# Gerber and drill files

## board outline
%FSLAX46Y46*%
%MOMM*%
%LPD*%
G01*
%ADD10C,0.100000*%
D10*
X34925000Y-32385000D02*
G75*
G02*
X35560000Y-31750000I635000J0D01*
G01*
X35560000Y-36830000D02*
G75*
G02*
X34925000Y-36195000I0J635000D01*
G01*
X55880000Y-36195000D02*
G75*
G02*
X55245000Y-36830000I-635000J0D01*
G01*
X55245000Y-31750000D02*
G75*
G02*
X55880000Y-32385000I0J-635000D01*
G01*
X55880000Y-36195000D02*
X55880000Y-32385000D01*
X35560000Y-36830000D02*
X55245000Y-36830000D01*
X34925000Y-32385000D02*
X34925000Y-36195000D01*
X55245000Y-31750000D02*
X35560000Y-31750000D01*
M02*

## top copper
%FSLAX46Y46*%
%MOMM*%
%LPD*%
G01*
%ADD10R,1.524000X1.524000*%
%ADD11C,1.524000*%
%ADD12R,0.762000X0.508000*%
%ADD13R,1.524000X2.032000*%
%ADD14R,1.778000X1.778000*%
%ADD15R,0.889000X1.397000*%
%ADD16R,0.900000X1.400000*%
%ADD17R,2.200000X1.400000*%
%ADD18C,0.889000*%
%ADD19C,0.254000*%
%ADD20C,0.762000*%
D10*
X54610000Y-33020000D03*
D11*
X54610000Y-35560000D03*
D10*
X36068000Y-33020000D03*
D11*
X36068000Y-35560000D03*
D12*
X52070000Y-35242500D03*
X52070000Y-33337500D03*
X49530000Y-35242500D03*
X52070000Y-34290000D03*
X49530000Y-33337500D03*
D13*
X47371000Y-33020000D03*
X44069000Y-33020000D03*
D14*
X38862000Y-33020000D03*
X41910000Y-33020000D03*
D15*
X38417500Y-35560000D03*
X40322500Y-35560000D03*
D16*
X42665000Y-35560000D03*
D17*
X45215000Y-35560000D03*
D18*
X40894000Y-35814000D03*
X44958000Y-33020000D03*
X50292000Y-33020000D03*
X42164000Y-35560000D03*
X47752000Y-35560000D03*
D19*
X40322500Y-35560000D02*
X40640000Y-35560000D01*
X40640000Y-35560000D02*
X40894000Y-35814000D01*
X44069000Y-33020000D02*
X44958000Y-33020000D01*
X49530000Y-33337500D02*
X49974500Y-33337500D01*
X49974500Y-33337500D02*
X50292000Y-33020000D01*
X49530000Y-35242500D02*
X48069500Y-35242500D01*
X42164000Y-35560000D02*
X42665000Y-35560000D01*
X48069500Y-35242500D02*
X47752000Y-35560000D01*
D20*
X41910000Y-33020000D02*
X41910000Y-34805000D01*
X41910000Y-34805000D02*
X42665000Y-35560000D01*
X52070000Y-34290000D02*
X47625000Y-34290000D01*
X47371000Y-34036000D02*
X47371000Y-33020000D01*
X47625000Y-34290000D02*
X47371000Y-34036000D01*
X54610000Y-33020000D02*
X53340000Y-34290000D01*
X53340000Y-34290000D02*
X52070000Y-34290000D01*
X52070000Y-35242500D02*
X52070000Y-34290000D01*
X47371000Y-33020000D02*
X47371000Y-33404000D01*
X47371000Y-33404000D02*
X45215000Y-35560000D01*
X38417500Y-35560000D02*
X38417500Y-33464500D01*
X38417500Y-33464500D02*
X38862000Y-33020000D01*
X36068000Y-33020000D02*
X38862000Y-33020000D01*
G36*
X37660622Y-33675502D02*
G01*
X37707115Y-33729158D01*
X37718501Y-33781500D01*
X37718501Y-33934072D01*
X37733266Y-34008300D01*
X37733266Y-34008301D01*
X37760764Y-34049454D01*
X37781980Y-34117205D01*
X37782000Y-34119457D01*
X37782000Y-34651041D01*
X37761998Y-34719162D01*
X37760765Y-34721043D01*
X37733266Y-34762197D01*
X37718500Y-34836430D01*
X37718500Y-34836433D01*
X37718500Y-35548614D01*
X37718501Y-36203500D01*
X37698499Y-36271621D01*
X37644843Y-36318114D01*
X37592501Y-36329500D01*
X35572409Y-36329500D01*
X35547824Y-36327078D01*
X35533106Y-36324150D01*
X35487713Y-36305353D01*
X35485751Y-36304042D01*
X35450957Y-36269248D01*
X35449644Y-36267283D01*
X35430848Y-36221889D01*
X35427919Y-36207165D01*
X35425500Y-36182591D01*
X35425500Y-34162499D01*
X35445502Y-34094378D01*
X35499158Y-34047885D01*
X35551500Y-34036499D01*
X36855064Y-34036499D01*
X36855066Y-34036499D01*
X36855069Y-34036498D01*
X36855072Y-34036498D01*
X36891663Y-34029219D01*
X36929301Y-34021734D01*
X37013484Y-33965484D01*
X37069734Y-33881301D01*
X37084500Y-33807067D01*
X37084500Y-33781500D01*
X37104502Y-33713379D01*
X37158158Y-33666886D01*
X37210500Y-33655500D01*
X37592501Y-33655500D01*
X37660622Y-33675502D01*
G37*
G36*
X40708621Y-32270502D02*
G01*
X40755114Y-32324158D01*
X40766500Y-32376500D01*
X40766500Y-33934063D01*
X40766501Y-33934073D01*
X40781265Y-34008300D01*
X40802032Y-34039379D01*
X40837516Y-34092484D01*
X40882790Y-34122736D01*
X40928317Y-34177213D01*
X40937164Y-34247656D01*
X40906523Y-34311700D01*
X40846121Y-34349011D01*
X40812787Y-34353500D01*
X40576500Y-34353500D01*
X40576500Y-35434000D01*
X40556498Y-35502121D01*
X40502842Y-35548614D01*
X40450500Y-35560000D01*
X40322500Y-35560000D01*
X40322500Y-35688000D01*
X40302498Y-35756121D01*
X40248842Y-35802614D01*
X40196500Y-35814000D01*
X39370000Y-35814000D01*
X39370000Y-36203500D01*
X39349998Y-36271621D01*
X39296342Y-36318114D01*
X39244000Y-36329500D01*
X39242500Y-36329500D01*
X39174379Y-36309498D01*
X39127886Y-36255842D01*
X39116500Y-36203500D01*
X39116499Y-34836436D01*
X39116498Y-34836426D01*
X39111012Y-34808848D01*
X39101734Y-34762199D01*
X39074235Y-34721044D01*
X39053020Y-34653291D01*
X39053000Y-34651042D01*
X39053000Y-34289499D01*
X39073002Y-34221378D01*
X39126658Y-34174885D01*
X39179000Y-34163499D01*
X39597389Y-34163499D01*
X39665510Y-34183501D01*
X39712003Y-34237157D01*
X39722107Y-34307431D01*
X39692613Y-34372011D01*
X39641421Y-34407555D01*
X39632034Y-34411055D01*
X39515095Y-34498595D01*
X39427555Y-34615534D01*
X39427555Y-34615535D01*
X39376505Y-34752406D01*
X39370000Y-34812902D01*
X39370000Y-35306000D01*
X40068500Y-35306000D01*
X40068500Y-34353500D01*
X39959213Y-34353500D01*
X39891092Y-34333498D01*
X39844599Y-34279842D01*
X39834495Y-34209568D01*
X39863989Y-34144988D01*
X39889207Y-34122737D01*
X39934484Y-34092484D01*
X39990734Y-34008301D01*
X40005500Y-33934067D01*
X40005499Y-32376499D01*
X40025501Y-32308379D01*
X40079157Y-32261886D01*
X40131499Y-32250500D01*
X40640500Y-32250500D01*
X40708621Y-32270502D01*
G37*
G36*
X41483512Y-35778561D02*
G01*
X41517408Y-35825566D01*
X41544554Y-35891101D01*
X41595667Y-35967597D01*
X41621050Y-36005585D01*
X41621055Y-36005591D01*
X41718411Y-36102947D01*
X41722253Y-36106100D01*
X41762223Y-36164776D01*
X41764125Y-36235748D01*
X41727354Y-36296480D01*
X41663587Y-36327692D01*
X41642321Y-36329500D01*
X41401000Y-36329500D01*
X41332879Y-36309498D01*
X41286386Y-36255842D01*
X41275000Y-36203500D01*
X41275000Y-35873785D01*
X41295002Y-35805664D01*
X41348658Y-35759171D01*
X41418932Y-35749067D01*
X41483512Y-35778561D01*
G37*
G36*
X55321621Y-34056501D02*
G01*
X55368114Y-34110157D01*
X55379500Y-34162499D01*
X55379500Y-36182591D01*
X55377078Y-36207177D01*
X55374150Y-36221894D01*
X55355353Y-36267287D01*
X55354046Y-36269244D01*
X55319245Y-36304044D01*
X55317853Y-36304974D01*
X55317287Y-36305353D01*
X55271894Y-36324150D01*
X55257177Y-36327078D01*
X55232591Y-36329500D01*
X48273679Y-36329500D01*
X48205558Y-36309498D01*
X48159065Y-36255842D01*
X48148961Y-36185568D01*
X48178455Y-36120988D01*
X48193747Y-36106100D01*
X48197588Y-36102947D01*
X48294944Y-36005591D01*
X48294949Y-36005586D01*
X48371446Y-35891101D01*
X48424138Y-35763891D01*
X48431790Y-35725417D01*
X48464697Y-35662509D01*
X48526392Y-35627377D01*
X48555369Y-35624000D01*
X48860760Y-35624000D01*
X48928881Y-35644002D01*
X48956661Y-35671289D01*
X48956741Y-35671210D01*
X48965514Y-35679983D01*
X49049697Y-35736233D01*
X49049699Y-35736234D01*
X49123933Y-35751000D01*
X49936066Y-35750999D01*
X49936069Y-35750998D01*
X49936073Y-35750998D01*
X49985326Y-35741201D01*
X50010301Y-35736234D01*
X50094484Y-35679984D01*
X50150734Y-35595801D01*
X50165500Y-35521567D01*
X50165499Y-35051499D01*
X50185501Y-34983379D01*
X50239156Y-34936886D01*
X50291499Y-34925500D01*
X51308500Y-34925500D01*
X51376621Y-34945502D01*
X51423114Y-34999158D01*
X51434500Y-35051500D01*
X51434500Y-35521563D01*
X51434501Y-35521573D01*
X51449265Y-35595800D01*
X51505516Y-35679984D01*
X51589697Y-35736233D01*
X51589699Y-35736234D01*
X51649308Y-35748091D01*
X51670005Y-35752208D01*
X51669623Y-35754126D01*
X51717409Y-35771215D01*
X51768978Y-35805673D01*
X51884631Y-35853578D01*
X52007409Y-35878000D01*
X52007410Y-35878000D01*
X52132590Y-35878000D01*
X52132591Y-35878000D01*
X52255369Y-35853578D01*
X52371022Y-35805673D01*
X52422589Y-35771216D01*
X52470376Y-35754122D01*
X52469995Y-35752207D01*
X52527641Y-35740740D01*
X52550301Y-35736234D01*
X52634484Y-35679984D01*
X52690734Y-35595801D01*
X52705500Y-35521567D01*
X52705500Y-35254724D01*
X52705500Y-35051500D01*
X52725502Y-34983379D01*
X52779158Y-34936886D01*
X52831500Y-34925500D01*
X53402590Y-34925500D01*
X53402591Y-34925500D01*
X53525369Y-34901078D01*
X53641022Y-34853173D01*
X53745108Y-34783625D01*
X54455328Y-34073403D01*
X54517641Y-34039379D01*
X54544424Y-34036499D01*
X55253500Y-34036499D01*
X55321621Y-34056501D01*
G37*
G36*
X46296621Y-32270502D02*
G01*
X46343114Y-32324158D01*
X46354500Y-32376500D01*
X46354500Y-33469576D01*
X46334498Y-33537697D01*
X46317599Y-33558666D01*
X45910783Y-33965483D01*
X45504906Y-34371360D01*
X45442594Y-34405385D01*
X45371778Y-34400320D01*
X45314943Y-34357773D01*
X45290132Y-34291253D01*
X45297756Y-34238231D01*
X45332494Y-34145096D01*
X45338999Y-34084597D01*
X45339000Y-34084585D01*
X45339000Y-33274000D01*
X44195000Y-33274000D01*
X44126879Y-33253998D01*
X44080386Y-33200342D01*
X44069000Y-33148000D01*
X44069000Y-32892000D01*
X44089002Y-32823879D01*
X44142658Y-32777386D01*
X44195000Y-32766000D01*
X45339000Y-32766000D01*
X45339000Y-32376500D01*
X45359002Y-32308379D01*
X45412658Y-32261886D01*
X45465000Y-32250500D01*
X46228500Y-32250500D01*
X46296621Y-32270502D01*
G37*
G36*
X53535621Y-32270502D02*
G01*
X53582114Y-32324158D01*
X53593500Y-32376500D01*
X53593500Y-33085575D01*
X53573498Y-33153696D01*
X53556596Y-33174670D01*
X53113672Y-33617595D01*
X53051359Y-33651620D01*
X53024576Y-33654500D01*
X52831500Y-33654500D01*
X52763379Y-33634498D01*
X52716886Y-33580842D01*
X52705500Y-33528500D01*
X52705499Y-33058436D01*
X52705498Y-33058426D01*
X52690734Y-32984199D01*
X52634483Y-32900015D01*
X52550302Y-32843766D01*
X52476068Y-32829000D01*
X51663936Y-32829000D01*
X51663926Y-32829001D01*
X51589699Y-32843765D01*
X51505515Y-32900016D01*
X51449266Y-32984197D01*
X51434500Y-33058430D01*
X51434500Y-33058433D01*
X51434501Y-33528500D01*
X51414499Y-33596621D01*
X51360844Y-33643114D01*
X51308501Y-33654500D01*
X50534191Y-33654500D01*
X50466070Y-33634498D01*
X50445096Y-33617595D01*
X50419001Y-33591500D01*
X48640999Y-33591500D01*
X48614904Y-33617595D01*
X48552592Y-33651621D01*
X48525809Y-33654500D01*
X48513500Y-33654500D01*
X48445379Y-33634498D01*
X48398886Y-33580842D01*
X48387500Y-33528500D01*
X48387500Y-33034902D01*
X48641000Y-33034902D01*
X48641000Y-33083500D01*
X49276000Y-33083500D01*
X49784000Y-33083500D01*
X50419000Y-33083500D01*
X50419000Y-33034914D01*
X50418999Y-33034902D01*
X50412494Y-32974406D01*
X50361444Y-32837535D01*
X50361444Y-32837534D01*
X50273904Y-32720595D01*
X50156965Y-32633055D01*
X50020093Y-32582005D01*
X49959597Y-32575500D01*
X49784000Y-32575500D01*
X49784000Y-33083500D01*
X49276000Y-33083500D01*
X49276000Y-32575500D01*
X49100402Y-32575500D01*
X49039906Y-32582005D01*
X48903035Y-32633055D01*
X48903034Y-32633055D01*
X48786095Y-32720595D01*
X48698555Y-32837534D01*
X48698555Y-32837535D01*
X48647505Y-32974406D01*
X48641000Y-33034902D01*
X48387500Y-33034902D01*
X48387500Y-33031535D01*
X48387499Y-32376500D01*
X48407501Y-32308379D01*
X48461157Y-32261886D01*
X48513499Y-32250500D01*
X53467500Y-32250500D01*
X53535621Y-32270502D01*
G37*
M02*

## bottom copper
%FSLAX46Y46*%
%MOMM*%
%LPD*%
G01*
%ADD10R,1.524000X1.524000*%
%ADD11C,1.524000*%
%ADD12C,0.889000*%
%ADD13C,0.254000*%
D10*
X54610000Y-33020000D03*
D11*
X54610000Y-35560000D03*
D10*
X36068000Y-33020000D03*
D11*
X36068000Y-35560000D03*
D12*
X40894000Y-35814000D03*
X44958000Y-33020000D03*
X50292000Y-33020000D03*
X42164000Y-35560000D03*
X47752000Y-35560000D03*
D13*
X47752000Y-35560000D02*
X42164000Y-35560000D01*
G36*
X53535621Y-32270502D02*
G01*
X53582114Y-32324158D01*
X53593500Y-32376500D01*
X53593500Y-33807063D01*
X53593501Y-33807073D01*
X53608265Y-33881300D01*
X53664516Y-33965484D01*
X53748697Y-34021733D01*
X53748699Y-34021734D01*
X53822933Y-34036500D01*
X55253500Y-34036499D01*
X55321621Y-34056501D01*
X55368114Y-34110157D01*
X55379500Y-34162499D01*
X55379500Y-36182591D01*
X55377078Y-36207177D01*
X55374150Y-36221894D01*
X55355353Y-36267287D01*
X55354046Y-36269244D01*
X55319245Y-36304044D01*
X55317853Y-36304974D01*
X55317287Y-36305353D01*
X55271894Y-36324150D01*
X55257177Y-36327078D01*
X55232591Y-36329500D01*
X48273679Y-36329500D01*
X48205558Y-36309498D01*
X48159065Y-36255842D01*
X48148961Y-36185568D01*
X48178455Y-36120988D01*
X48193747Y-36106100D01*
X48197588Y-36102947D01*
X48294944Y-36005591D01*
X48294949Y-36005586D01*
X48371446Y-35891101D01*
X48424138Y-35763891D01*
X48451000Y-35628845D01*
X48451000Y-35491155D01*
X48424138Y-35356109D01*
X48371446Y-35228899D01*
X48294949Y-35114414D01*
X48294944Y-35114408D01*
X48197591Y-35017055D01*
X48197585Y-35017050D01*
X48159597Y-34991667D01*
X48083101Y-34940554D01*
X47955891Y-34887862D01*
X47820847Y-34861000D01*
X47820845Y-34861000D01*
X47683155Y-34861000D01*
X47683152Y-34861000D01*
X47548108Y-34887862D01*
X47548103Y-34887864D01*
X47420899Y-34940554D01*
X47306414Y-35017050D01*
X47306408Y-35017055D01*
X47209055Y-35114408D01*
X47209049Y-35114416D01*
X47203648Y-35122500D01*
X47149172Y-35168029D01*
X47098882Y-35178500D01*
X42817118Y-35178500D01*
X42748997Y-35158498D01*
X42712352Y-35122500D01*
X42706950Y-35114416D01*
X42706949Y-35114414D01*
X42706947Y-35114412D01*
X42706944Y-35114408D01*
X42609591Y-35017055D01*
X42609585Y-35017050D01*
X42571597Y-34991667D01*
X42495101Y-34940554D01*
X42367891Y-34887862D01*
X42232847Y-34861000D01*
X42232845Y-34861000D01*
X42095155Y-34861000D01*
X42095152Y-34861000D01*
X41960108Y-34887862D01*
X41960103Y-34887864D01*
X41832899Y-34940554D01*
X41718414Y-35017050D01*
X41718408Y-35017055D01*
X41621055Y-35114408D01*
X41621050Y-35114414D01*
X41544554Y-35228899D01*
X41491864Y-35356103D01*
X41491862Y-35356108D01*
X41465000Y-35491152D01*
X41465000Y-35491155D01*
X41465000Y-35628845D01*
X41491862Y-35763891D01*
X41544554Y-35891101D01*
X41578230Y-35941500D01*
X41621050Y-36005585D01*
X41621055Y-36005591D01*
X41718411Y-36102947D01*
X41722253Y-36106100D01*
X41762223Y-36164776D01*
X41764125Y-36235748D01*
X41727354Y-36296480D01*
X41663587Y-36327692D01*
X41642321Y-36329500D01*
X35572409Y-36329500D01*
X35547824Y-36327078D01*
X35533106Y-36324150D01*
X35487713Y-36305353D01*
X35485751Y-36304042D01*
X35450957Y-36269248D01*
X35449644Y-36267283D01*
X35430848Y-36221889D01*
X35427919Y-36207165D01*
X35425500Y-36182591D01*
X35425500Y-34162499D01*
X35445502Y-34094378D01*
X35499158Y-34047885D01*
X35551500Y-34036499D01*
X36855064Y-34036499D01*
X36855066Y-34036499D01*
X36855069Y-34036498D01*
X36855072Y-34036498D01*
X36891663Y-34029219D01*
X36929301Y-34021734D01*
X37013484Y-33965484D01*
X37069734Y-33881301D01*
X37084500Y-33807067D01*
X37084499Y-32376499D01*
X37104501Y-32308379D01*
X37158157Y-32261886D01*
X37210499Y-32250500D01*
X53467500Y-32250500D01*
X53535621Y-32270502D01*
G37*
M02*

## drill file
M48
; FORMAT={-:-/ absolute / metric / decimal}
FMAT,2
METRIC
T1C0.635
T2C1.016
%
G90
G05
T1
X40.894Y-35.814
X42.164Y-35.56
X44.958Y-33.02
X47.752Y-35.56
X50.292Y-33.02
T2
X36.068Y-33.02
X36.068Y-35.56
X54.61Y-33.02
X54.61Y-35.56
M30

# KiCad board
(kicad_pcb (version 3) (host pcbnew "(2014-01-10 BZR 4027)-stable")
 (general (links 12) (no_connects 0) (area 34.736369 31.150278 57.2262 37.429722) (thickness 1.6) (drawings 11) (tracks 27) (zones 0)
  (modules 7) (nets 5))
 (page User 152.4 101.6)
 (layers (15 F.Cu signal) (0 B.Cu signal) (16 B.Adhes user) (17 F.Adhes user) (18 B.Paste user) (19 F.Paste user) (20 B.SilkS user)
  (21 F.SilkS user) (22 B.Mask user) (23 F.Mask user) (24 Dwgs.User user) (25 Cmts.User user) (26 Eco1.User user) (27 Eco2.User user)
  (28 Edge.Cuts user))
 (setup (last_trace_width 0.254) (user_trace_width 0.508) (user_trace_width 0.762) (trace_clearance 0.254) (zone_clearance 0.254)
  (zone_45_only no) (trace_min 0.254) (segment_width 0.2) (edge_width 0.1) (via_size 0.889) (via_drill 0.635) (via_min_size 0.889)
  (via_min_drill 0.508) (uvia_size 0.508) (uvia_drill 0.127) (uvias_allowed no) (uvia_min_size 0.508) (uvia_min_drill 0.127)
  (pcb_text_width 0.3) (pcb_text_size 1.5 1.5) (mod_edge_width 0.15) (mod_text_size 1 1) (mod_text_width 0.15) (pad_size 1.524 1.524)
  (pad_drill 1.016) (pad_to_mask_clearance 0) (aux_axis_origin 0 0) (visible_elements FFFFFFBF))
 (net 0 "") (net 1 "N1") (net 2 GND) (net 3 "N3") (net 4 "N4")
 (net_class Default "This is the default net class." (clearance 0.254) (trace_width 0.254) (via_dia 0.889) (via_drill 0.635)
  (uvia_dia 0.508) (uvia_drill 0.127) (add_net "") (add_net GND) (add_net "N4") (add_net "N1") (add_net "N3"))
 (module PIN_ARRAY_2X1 (layer F.Cu) (at 54.61 34.29 270)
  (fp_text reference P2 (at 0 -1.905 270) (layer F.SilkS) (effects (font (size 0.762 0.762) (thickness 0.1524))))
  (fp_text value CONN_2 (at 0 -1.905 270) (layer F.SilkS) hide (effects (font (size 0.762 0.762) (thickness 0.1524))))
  (pad 1 thru_hole rect (at -1.27 0 270) (size 1.524 1.524) (drill 1.016) (layers *.Cu *.Mask F.SilkS) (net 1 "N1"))
  (pad 2 thru_hole circle (at 1.27 0 270) (size 1.524 1.524) (drill 1.016) (layers *.Cu *.Mask F.SilkS) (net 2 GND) (zone_connect 2)))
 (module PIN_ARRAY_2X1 (layer F.Cu) (at 36.068 34.29 270)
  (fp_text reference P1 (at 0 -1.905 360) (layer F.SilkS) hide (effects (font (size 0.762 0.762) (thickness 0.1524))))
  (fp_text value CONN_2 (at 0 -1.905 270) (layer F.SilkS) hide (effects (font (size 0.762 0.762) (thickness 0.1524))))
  (pad 1 thru_hole rect (at -1.27 0 270) (size 1.524 1.524) (drill 1.016) (layers *.Cu *.Mask F.SilkS) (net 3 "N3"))
  (pad 2 thru_hole circle (at 1.27 0 270) (size 1.524 1.524) (drill 1.016) (layers *.Cu *.Mask F.SilkS) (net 2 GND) (zone_connect 2)))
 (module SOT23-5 (layer F.Cu) (at 50.8 34.29 90)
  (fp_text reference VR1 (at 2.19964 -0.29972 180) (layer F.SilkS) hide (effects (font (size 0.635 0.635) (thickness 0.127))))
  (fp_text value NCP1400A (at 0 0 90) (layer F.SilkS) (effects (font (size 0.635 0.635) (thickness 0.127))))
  (pad 1 smd rect (at -0.9525 1.27 90) (size 0.508 0.762) (layers F.Cu F.Paste F.Mask) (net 1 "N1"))
  (pad 3 smd rect (at 0.9525 1.27 90) (size 0.508 0.762) (layers F.Cu F.Paste F.Mask))
  (pad 5 smd rect (at -0.9525 -1.27 90) (size 0.508 0.762) (layers F.Cu F.Paste F.Mask) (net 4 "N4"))
  (pad 2 smd rect (at 0 1.27 90) (size 0.508 0.762) (layers F.Cu F.Paste F.Mask) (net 1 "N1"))
  (pad 4 smd rect (at 0.9525 -1.27 90) (size 0.508 0.762) (layers F.Cu F.Paste F.Mask) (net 2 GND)))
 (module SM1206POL (layer F.Cu) (at 45.72 33.02 180)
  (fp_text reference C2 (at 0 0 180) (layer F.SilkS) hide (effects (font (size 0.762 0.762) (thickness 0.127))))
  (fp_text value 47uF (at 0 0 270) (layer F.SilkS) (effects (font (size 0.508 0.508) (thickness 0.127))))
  (pad 1 smd rect (at -1.651 0 180) (size 1.524 2.032) (layers F.Cu F.Paste F.Mask) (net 1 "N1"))
  (pad 2 smd rect (at 1.651 0 180) (size 1.524 2.032) (layers F.Cu F.Paste F.Mask) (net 2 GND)))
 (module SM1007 (layer F.Cu) (at 40.386 33.02)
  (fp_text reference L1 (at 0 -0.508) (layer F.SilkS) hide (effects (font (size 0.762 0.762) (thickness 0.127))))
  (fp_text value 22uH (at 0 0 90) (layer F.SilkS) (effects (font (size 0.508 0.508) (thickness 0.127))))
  (pad 1 smd rect (at -1.524 0) (size 1.778 1.778) (layers F.Cu F.Paste F.Mask) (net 3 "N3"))
  (pad 2 smd rect (at 1.524 0) (size 1.778 1.778) (layers F.Cu F.Paste F.Mask) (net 4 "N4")))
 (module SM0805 (layer F.Cu) (at 39.37 35.56)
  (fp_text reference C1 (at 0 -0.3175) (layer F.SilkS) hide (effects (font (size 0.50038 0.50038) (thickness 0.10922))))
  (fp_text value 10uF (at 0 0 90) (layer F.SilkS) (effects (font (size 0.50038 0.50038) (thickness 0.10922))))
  (pad 1 smd rect (at -0.9525 0) (size 0.889 1.397) (layers F.Cu F.Paste F.Mask) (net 3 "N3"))
  (pad 2 smd rect (at 0.9525 0) (size 0.889 1.397) (layers F.Cu F.Paste F.Mask) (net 2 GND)))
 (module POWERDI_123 (layer F.Cu) (at 43.815 35.56)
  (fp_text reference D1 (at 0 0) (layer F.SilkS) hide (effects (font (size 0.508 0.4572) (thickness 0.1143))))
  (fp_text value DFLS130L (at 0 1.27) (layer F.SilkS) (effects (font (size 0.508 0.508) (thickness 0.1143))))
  (pad 1 smd rect (at -1.15 0) (size 0.9 1.4) (layers F.Cu F.Paste F.Mask) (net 4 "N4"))
  (pad 2 smd rect (at 1.4 0) (size 2.2 1.4) (layers F.Cu F.Paste F.Mask) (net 1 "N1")))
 (gr_arc (start 35.56 32.385) (end 34.925 32.385) (angle 90) (layer Edge.Cuts) (width 0.1))
 (gr_arc (start 35.56 36.195) (end 35.56 36.83) (angle 90) (layer Edge.Cuts) (width 0.1))
 (gr_arc (start 55.245 36.195) (end 55.88 36.195) (angle 90) (layer Edge.Cuts) (width 0.1))
 (gr_arc (start 55.245 32.385) (end 55.245 31.75) (angle 90) (layer Edge.Cuts) (width 0.1))
 (gr_line (start 55.88 36.195) (end 55.88 32.385) (angle 90) (layer Edge.Cuts) (width 0.1))
 (gr_line (start 35.56 36.83) (end 55.245 36.83) (angle 90) (layer Edge.Cuts) (width 0.1))
 (gr_line (start 34.925 32.385) (end 34.925 36.195) (angle 90) (layer Edge.Cuts) (width 0.1))
 (gr_line (start 55.245 31.75) (end 35.56 31.75) (angle 90) (layer Edge.Cuts) (width 0.1))
 (segment (start 40.3225 35.56) (end 40.64 35.56) (width 0.254) (layer F.Cu) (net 2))
 (via (at 40.894 35.814) (size 0.889) (layers F.Cu B.Cu) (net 2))
 (segment (start 40.64 35.56) (end 40.894 35.814) (width 0.254) (layer F.Cu) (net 2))
 (segment (start 44.069 33.02) (end 44.958 33.02) (width 0.254) (layer F.Cu) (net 2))
 (via (at 44.958 33.02) (size 0.889) (layers F.Cu B.Cu) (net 2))
 (segment (start 49.53 33.3375) (end 49.9745 33.3375) (width 0.254) (layer F.Cu) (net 2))
 (via (at 50.292 33.02) (size 0.889) (layers F.Cu B.Cu) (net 2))
 (segment (start 49.9745 33.3375) (end 50.292 33.02) (width 0.254) (layer F.Cu) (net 2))
 (segment (start 49.53 35.2425) (end 48.0695 35.2425) (width 0.254) (layer F.Cu) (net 4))
 (segment (start 42.164 35.56) (end 42.665 35.56) (width 0.254) (layer F.Cu) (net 4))
 (via (at 42.164 35.56) (size 0.889) (layers F.Cu B.Cu) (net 4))
 (segment (start 47.752 35.56) (end 42.164 35.56) (width 0.254) (layer B.Cu) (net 4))
 (via (at 47.752 35.56) (size 0.889) (layers F.Cu B.Cu) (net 4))
 (segment (start 48.0695 35.2425) (end 47.752 35.56) (width 0.254) (layer F.Cu) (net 4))
 (segment (start 41.91 33.02) (end 41.91 34.805) (width 0.762) (layer F.Cu) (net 4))
 (segment (start 41.91 34.805) (end 42.665 35.56) (width 0.762) (layer F.Cu) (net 4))
 (segment (start 52.07 34.29) (end 47.625 34.29) (width 0.762) (layer F.Cu) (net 1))
 (segment (start 47.371 34.036) (end 47.371 33.02) (width 0.762) (layer F.Cu) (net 1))
 (segment (start 47.625 34.29) (end 47.371 34.036) (width 0.762) (layer F.Cu) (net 1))
 (segment (start 54.61 33.02) (end 53.34 34.29) (width 0.762) (layer F.Cu) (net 1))
 (segment (start 53.34 34.29) (end 52.07 34.29) (width 0.762) (layer F.Cu) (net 1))
 (segment (start 52.07 35.2425) (end 52.07 34.29) (width 0.762) (layer F.Cu) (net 1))
 (segment (start 47.371 33.02) (end 47.371 33.404) (width 0.762) (layer F.Cu) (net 1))
 (segment (start 47.371 33.404) (end 45.215 35.56) (width 0.762) (layer F.Cu) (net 1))
 (segment (start 38.4175 35.56) (end 38.4175 33.4645) (width 0.762) (layer F.Cu) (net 3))
 (segment (start 38.4175 33.4645) (end 38.862 33.02) (width 0.762) (layer F.Cu) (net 3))
 (segment (start 36.068 33.02) (end 38.862 33.02) (width 0.762) (layer F.Cu) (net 3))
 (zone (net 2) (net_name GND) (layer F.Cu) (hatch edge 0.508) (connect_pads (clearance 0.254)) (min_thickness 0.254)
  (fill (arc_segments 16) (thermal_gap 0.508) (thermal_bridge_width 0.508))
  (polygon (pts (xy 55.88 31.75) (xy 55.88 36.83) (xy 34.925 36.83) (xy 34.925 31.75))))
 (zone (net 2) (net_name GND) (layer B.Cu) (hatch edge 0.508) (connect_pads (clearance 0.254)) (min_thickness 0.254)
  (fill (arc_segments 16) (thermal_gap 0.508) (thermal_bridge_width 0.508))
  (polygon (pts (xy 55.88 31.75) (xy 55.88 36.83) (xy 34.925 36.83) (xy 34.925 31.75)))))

